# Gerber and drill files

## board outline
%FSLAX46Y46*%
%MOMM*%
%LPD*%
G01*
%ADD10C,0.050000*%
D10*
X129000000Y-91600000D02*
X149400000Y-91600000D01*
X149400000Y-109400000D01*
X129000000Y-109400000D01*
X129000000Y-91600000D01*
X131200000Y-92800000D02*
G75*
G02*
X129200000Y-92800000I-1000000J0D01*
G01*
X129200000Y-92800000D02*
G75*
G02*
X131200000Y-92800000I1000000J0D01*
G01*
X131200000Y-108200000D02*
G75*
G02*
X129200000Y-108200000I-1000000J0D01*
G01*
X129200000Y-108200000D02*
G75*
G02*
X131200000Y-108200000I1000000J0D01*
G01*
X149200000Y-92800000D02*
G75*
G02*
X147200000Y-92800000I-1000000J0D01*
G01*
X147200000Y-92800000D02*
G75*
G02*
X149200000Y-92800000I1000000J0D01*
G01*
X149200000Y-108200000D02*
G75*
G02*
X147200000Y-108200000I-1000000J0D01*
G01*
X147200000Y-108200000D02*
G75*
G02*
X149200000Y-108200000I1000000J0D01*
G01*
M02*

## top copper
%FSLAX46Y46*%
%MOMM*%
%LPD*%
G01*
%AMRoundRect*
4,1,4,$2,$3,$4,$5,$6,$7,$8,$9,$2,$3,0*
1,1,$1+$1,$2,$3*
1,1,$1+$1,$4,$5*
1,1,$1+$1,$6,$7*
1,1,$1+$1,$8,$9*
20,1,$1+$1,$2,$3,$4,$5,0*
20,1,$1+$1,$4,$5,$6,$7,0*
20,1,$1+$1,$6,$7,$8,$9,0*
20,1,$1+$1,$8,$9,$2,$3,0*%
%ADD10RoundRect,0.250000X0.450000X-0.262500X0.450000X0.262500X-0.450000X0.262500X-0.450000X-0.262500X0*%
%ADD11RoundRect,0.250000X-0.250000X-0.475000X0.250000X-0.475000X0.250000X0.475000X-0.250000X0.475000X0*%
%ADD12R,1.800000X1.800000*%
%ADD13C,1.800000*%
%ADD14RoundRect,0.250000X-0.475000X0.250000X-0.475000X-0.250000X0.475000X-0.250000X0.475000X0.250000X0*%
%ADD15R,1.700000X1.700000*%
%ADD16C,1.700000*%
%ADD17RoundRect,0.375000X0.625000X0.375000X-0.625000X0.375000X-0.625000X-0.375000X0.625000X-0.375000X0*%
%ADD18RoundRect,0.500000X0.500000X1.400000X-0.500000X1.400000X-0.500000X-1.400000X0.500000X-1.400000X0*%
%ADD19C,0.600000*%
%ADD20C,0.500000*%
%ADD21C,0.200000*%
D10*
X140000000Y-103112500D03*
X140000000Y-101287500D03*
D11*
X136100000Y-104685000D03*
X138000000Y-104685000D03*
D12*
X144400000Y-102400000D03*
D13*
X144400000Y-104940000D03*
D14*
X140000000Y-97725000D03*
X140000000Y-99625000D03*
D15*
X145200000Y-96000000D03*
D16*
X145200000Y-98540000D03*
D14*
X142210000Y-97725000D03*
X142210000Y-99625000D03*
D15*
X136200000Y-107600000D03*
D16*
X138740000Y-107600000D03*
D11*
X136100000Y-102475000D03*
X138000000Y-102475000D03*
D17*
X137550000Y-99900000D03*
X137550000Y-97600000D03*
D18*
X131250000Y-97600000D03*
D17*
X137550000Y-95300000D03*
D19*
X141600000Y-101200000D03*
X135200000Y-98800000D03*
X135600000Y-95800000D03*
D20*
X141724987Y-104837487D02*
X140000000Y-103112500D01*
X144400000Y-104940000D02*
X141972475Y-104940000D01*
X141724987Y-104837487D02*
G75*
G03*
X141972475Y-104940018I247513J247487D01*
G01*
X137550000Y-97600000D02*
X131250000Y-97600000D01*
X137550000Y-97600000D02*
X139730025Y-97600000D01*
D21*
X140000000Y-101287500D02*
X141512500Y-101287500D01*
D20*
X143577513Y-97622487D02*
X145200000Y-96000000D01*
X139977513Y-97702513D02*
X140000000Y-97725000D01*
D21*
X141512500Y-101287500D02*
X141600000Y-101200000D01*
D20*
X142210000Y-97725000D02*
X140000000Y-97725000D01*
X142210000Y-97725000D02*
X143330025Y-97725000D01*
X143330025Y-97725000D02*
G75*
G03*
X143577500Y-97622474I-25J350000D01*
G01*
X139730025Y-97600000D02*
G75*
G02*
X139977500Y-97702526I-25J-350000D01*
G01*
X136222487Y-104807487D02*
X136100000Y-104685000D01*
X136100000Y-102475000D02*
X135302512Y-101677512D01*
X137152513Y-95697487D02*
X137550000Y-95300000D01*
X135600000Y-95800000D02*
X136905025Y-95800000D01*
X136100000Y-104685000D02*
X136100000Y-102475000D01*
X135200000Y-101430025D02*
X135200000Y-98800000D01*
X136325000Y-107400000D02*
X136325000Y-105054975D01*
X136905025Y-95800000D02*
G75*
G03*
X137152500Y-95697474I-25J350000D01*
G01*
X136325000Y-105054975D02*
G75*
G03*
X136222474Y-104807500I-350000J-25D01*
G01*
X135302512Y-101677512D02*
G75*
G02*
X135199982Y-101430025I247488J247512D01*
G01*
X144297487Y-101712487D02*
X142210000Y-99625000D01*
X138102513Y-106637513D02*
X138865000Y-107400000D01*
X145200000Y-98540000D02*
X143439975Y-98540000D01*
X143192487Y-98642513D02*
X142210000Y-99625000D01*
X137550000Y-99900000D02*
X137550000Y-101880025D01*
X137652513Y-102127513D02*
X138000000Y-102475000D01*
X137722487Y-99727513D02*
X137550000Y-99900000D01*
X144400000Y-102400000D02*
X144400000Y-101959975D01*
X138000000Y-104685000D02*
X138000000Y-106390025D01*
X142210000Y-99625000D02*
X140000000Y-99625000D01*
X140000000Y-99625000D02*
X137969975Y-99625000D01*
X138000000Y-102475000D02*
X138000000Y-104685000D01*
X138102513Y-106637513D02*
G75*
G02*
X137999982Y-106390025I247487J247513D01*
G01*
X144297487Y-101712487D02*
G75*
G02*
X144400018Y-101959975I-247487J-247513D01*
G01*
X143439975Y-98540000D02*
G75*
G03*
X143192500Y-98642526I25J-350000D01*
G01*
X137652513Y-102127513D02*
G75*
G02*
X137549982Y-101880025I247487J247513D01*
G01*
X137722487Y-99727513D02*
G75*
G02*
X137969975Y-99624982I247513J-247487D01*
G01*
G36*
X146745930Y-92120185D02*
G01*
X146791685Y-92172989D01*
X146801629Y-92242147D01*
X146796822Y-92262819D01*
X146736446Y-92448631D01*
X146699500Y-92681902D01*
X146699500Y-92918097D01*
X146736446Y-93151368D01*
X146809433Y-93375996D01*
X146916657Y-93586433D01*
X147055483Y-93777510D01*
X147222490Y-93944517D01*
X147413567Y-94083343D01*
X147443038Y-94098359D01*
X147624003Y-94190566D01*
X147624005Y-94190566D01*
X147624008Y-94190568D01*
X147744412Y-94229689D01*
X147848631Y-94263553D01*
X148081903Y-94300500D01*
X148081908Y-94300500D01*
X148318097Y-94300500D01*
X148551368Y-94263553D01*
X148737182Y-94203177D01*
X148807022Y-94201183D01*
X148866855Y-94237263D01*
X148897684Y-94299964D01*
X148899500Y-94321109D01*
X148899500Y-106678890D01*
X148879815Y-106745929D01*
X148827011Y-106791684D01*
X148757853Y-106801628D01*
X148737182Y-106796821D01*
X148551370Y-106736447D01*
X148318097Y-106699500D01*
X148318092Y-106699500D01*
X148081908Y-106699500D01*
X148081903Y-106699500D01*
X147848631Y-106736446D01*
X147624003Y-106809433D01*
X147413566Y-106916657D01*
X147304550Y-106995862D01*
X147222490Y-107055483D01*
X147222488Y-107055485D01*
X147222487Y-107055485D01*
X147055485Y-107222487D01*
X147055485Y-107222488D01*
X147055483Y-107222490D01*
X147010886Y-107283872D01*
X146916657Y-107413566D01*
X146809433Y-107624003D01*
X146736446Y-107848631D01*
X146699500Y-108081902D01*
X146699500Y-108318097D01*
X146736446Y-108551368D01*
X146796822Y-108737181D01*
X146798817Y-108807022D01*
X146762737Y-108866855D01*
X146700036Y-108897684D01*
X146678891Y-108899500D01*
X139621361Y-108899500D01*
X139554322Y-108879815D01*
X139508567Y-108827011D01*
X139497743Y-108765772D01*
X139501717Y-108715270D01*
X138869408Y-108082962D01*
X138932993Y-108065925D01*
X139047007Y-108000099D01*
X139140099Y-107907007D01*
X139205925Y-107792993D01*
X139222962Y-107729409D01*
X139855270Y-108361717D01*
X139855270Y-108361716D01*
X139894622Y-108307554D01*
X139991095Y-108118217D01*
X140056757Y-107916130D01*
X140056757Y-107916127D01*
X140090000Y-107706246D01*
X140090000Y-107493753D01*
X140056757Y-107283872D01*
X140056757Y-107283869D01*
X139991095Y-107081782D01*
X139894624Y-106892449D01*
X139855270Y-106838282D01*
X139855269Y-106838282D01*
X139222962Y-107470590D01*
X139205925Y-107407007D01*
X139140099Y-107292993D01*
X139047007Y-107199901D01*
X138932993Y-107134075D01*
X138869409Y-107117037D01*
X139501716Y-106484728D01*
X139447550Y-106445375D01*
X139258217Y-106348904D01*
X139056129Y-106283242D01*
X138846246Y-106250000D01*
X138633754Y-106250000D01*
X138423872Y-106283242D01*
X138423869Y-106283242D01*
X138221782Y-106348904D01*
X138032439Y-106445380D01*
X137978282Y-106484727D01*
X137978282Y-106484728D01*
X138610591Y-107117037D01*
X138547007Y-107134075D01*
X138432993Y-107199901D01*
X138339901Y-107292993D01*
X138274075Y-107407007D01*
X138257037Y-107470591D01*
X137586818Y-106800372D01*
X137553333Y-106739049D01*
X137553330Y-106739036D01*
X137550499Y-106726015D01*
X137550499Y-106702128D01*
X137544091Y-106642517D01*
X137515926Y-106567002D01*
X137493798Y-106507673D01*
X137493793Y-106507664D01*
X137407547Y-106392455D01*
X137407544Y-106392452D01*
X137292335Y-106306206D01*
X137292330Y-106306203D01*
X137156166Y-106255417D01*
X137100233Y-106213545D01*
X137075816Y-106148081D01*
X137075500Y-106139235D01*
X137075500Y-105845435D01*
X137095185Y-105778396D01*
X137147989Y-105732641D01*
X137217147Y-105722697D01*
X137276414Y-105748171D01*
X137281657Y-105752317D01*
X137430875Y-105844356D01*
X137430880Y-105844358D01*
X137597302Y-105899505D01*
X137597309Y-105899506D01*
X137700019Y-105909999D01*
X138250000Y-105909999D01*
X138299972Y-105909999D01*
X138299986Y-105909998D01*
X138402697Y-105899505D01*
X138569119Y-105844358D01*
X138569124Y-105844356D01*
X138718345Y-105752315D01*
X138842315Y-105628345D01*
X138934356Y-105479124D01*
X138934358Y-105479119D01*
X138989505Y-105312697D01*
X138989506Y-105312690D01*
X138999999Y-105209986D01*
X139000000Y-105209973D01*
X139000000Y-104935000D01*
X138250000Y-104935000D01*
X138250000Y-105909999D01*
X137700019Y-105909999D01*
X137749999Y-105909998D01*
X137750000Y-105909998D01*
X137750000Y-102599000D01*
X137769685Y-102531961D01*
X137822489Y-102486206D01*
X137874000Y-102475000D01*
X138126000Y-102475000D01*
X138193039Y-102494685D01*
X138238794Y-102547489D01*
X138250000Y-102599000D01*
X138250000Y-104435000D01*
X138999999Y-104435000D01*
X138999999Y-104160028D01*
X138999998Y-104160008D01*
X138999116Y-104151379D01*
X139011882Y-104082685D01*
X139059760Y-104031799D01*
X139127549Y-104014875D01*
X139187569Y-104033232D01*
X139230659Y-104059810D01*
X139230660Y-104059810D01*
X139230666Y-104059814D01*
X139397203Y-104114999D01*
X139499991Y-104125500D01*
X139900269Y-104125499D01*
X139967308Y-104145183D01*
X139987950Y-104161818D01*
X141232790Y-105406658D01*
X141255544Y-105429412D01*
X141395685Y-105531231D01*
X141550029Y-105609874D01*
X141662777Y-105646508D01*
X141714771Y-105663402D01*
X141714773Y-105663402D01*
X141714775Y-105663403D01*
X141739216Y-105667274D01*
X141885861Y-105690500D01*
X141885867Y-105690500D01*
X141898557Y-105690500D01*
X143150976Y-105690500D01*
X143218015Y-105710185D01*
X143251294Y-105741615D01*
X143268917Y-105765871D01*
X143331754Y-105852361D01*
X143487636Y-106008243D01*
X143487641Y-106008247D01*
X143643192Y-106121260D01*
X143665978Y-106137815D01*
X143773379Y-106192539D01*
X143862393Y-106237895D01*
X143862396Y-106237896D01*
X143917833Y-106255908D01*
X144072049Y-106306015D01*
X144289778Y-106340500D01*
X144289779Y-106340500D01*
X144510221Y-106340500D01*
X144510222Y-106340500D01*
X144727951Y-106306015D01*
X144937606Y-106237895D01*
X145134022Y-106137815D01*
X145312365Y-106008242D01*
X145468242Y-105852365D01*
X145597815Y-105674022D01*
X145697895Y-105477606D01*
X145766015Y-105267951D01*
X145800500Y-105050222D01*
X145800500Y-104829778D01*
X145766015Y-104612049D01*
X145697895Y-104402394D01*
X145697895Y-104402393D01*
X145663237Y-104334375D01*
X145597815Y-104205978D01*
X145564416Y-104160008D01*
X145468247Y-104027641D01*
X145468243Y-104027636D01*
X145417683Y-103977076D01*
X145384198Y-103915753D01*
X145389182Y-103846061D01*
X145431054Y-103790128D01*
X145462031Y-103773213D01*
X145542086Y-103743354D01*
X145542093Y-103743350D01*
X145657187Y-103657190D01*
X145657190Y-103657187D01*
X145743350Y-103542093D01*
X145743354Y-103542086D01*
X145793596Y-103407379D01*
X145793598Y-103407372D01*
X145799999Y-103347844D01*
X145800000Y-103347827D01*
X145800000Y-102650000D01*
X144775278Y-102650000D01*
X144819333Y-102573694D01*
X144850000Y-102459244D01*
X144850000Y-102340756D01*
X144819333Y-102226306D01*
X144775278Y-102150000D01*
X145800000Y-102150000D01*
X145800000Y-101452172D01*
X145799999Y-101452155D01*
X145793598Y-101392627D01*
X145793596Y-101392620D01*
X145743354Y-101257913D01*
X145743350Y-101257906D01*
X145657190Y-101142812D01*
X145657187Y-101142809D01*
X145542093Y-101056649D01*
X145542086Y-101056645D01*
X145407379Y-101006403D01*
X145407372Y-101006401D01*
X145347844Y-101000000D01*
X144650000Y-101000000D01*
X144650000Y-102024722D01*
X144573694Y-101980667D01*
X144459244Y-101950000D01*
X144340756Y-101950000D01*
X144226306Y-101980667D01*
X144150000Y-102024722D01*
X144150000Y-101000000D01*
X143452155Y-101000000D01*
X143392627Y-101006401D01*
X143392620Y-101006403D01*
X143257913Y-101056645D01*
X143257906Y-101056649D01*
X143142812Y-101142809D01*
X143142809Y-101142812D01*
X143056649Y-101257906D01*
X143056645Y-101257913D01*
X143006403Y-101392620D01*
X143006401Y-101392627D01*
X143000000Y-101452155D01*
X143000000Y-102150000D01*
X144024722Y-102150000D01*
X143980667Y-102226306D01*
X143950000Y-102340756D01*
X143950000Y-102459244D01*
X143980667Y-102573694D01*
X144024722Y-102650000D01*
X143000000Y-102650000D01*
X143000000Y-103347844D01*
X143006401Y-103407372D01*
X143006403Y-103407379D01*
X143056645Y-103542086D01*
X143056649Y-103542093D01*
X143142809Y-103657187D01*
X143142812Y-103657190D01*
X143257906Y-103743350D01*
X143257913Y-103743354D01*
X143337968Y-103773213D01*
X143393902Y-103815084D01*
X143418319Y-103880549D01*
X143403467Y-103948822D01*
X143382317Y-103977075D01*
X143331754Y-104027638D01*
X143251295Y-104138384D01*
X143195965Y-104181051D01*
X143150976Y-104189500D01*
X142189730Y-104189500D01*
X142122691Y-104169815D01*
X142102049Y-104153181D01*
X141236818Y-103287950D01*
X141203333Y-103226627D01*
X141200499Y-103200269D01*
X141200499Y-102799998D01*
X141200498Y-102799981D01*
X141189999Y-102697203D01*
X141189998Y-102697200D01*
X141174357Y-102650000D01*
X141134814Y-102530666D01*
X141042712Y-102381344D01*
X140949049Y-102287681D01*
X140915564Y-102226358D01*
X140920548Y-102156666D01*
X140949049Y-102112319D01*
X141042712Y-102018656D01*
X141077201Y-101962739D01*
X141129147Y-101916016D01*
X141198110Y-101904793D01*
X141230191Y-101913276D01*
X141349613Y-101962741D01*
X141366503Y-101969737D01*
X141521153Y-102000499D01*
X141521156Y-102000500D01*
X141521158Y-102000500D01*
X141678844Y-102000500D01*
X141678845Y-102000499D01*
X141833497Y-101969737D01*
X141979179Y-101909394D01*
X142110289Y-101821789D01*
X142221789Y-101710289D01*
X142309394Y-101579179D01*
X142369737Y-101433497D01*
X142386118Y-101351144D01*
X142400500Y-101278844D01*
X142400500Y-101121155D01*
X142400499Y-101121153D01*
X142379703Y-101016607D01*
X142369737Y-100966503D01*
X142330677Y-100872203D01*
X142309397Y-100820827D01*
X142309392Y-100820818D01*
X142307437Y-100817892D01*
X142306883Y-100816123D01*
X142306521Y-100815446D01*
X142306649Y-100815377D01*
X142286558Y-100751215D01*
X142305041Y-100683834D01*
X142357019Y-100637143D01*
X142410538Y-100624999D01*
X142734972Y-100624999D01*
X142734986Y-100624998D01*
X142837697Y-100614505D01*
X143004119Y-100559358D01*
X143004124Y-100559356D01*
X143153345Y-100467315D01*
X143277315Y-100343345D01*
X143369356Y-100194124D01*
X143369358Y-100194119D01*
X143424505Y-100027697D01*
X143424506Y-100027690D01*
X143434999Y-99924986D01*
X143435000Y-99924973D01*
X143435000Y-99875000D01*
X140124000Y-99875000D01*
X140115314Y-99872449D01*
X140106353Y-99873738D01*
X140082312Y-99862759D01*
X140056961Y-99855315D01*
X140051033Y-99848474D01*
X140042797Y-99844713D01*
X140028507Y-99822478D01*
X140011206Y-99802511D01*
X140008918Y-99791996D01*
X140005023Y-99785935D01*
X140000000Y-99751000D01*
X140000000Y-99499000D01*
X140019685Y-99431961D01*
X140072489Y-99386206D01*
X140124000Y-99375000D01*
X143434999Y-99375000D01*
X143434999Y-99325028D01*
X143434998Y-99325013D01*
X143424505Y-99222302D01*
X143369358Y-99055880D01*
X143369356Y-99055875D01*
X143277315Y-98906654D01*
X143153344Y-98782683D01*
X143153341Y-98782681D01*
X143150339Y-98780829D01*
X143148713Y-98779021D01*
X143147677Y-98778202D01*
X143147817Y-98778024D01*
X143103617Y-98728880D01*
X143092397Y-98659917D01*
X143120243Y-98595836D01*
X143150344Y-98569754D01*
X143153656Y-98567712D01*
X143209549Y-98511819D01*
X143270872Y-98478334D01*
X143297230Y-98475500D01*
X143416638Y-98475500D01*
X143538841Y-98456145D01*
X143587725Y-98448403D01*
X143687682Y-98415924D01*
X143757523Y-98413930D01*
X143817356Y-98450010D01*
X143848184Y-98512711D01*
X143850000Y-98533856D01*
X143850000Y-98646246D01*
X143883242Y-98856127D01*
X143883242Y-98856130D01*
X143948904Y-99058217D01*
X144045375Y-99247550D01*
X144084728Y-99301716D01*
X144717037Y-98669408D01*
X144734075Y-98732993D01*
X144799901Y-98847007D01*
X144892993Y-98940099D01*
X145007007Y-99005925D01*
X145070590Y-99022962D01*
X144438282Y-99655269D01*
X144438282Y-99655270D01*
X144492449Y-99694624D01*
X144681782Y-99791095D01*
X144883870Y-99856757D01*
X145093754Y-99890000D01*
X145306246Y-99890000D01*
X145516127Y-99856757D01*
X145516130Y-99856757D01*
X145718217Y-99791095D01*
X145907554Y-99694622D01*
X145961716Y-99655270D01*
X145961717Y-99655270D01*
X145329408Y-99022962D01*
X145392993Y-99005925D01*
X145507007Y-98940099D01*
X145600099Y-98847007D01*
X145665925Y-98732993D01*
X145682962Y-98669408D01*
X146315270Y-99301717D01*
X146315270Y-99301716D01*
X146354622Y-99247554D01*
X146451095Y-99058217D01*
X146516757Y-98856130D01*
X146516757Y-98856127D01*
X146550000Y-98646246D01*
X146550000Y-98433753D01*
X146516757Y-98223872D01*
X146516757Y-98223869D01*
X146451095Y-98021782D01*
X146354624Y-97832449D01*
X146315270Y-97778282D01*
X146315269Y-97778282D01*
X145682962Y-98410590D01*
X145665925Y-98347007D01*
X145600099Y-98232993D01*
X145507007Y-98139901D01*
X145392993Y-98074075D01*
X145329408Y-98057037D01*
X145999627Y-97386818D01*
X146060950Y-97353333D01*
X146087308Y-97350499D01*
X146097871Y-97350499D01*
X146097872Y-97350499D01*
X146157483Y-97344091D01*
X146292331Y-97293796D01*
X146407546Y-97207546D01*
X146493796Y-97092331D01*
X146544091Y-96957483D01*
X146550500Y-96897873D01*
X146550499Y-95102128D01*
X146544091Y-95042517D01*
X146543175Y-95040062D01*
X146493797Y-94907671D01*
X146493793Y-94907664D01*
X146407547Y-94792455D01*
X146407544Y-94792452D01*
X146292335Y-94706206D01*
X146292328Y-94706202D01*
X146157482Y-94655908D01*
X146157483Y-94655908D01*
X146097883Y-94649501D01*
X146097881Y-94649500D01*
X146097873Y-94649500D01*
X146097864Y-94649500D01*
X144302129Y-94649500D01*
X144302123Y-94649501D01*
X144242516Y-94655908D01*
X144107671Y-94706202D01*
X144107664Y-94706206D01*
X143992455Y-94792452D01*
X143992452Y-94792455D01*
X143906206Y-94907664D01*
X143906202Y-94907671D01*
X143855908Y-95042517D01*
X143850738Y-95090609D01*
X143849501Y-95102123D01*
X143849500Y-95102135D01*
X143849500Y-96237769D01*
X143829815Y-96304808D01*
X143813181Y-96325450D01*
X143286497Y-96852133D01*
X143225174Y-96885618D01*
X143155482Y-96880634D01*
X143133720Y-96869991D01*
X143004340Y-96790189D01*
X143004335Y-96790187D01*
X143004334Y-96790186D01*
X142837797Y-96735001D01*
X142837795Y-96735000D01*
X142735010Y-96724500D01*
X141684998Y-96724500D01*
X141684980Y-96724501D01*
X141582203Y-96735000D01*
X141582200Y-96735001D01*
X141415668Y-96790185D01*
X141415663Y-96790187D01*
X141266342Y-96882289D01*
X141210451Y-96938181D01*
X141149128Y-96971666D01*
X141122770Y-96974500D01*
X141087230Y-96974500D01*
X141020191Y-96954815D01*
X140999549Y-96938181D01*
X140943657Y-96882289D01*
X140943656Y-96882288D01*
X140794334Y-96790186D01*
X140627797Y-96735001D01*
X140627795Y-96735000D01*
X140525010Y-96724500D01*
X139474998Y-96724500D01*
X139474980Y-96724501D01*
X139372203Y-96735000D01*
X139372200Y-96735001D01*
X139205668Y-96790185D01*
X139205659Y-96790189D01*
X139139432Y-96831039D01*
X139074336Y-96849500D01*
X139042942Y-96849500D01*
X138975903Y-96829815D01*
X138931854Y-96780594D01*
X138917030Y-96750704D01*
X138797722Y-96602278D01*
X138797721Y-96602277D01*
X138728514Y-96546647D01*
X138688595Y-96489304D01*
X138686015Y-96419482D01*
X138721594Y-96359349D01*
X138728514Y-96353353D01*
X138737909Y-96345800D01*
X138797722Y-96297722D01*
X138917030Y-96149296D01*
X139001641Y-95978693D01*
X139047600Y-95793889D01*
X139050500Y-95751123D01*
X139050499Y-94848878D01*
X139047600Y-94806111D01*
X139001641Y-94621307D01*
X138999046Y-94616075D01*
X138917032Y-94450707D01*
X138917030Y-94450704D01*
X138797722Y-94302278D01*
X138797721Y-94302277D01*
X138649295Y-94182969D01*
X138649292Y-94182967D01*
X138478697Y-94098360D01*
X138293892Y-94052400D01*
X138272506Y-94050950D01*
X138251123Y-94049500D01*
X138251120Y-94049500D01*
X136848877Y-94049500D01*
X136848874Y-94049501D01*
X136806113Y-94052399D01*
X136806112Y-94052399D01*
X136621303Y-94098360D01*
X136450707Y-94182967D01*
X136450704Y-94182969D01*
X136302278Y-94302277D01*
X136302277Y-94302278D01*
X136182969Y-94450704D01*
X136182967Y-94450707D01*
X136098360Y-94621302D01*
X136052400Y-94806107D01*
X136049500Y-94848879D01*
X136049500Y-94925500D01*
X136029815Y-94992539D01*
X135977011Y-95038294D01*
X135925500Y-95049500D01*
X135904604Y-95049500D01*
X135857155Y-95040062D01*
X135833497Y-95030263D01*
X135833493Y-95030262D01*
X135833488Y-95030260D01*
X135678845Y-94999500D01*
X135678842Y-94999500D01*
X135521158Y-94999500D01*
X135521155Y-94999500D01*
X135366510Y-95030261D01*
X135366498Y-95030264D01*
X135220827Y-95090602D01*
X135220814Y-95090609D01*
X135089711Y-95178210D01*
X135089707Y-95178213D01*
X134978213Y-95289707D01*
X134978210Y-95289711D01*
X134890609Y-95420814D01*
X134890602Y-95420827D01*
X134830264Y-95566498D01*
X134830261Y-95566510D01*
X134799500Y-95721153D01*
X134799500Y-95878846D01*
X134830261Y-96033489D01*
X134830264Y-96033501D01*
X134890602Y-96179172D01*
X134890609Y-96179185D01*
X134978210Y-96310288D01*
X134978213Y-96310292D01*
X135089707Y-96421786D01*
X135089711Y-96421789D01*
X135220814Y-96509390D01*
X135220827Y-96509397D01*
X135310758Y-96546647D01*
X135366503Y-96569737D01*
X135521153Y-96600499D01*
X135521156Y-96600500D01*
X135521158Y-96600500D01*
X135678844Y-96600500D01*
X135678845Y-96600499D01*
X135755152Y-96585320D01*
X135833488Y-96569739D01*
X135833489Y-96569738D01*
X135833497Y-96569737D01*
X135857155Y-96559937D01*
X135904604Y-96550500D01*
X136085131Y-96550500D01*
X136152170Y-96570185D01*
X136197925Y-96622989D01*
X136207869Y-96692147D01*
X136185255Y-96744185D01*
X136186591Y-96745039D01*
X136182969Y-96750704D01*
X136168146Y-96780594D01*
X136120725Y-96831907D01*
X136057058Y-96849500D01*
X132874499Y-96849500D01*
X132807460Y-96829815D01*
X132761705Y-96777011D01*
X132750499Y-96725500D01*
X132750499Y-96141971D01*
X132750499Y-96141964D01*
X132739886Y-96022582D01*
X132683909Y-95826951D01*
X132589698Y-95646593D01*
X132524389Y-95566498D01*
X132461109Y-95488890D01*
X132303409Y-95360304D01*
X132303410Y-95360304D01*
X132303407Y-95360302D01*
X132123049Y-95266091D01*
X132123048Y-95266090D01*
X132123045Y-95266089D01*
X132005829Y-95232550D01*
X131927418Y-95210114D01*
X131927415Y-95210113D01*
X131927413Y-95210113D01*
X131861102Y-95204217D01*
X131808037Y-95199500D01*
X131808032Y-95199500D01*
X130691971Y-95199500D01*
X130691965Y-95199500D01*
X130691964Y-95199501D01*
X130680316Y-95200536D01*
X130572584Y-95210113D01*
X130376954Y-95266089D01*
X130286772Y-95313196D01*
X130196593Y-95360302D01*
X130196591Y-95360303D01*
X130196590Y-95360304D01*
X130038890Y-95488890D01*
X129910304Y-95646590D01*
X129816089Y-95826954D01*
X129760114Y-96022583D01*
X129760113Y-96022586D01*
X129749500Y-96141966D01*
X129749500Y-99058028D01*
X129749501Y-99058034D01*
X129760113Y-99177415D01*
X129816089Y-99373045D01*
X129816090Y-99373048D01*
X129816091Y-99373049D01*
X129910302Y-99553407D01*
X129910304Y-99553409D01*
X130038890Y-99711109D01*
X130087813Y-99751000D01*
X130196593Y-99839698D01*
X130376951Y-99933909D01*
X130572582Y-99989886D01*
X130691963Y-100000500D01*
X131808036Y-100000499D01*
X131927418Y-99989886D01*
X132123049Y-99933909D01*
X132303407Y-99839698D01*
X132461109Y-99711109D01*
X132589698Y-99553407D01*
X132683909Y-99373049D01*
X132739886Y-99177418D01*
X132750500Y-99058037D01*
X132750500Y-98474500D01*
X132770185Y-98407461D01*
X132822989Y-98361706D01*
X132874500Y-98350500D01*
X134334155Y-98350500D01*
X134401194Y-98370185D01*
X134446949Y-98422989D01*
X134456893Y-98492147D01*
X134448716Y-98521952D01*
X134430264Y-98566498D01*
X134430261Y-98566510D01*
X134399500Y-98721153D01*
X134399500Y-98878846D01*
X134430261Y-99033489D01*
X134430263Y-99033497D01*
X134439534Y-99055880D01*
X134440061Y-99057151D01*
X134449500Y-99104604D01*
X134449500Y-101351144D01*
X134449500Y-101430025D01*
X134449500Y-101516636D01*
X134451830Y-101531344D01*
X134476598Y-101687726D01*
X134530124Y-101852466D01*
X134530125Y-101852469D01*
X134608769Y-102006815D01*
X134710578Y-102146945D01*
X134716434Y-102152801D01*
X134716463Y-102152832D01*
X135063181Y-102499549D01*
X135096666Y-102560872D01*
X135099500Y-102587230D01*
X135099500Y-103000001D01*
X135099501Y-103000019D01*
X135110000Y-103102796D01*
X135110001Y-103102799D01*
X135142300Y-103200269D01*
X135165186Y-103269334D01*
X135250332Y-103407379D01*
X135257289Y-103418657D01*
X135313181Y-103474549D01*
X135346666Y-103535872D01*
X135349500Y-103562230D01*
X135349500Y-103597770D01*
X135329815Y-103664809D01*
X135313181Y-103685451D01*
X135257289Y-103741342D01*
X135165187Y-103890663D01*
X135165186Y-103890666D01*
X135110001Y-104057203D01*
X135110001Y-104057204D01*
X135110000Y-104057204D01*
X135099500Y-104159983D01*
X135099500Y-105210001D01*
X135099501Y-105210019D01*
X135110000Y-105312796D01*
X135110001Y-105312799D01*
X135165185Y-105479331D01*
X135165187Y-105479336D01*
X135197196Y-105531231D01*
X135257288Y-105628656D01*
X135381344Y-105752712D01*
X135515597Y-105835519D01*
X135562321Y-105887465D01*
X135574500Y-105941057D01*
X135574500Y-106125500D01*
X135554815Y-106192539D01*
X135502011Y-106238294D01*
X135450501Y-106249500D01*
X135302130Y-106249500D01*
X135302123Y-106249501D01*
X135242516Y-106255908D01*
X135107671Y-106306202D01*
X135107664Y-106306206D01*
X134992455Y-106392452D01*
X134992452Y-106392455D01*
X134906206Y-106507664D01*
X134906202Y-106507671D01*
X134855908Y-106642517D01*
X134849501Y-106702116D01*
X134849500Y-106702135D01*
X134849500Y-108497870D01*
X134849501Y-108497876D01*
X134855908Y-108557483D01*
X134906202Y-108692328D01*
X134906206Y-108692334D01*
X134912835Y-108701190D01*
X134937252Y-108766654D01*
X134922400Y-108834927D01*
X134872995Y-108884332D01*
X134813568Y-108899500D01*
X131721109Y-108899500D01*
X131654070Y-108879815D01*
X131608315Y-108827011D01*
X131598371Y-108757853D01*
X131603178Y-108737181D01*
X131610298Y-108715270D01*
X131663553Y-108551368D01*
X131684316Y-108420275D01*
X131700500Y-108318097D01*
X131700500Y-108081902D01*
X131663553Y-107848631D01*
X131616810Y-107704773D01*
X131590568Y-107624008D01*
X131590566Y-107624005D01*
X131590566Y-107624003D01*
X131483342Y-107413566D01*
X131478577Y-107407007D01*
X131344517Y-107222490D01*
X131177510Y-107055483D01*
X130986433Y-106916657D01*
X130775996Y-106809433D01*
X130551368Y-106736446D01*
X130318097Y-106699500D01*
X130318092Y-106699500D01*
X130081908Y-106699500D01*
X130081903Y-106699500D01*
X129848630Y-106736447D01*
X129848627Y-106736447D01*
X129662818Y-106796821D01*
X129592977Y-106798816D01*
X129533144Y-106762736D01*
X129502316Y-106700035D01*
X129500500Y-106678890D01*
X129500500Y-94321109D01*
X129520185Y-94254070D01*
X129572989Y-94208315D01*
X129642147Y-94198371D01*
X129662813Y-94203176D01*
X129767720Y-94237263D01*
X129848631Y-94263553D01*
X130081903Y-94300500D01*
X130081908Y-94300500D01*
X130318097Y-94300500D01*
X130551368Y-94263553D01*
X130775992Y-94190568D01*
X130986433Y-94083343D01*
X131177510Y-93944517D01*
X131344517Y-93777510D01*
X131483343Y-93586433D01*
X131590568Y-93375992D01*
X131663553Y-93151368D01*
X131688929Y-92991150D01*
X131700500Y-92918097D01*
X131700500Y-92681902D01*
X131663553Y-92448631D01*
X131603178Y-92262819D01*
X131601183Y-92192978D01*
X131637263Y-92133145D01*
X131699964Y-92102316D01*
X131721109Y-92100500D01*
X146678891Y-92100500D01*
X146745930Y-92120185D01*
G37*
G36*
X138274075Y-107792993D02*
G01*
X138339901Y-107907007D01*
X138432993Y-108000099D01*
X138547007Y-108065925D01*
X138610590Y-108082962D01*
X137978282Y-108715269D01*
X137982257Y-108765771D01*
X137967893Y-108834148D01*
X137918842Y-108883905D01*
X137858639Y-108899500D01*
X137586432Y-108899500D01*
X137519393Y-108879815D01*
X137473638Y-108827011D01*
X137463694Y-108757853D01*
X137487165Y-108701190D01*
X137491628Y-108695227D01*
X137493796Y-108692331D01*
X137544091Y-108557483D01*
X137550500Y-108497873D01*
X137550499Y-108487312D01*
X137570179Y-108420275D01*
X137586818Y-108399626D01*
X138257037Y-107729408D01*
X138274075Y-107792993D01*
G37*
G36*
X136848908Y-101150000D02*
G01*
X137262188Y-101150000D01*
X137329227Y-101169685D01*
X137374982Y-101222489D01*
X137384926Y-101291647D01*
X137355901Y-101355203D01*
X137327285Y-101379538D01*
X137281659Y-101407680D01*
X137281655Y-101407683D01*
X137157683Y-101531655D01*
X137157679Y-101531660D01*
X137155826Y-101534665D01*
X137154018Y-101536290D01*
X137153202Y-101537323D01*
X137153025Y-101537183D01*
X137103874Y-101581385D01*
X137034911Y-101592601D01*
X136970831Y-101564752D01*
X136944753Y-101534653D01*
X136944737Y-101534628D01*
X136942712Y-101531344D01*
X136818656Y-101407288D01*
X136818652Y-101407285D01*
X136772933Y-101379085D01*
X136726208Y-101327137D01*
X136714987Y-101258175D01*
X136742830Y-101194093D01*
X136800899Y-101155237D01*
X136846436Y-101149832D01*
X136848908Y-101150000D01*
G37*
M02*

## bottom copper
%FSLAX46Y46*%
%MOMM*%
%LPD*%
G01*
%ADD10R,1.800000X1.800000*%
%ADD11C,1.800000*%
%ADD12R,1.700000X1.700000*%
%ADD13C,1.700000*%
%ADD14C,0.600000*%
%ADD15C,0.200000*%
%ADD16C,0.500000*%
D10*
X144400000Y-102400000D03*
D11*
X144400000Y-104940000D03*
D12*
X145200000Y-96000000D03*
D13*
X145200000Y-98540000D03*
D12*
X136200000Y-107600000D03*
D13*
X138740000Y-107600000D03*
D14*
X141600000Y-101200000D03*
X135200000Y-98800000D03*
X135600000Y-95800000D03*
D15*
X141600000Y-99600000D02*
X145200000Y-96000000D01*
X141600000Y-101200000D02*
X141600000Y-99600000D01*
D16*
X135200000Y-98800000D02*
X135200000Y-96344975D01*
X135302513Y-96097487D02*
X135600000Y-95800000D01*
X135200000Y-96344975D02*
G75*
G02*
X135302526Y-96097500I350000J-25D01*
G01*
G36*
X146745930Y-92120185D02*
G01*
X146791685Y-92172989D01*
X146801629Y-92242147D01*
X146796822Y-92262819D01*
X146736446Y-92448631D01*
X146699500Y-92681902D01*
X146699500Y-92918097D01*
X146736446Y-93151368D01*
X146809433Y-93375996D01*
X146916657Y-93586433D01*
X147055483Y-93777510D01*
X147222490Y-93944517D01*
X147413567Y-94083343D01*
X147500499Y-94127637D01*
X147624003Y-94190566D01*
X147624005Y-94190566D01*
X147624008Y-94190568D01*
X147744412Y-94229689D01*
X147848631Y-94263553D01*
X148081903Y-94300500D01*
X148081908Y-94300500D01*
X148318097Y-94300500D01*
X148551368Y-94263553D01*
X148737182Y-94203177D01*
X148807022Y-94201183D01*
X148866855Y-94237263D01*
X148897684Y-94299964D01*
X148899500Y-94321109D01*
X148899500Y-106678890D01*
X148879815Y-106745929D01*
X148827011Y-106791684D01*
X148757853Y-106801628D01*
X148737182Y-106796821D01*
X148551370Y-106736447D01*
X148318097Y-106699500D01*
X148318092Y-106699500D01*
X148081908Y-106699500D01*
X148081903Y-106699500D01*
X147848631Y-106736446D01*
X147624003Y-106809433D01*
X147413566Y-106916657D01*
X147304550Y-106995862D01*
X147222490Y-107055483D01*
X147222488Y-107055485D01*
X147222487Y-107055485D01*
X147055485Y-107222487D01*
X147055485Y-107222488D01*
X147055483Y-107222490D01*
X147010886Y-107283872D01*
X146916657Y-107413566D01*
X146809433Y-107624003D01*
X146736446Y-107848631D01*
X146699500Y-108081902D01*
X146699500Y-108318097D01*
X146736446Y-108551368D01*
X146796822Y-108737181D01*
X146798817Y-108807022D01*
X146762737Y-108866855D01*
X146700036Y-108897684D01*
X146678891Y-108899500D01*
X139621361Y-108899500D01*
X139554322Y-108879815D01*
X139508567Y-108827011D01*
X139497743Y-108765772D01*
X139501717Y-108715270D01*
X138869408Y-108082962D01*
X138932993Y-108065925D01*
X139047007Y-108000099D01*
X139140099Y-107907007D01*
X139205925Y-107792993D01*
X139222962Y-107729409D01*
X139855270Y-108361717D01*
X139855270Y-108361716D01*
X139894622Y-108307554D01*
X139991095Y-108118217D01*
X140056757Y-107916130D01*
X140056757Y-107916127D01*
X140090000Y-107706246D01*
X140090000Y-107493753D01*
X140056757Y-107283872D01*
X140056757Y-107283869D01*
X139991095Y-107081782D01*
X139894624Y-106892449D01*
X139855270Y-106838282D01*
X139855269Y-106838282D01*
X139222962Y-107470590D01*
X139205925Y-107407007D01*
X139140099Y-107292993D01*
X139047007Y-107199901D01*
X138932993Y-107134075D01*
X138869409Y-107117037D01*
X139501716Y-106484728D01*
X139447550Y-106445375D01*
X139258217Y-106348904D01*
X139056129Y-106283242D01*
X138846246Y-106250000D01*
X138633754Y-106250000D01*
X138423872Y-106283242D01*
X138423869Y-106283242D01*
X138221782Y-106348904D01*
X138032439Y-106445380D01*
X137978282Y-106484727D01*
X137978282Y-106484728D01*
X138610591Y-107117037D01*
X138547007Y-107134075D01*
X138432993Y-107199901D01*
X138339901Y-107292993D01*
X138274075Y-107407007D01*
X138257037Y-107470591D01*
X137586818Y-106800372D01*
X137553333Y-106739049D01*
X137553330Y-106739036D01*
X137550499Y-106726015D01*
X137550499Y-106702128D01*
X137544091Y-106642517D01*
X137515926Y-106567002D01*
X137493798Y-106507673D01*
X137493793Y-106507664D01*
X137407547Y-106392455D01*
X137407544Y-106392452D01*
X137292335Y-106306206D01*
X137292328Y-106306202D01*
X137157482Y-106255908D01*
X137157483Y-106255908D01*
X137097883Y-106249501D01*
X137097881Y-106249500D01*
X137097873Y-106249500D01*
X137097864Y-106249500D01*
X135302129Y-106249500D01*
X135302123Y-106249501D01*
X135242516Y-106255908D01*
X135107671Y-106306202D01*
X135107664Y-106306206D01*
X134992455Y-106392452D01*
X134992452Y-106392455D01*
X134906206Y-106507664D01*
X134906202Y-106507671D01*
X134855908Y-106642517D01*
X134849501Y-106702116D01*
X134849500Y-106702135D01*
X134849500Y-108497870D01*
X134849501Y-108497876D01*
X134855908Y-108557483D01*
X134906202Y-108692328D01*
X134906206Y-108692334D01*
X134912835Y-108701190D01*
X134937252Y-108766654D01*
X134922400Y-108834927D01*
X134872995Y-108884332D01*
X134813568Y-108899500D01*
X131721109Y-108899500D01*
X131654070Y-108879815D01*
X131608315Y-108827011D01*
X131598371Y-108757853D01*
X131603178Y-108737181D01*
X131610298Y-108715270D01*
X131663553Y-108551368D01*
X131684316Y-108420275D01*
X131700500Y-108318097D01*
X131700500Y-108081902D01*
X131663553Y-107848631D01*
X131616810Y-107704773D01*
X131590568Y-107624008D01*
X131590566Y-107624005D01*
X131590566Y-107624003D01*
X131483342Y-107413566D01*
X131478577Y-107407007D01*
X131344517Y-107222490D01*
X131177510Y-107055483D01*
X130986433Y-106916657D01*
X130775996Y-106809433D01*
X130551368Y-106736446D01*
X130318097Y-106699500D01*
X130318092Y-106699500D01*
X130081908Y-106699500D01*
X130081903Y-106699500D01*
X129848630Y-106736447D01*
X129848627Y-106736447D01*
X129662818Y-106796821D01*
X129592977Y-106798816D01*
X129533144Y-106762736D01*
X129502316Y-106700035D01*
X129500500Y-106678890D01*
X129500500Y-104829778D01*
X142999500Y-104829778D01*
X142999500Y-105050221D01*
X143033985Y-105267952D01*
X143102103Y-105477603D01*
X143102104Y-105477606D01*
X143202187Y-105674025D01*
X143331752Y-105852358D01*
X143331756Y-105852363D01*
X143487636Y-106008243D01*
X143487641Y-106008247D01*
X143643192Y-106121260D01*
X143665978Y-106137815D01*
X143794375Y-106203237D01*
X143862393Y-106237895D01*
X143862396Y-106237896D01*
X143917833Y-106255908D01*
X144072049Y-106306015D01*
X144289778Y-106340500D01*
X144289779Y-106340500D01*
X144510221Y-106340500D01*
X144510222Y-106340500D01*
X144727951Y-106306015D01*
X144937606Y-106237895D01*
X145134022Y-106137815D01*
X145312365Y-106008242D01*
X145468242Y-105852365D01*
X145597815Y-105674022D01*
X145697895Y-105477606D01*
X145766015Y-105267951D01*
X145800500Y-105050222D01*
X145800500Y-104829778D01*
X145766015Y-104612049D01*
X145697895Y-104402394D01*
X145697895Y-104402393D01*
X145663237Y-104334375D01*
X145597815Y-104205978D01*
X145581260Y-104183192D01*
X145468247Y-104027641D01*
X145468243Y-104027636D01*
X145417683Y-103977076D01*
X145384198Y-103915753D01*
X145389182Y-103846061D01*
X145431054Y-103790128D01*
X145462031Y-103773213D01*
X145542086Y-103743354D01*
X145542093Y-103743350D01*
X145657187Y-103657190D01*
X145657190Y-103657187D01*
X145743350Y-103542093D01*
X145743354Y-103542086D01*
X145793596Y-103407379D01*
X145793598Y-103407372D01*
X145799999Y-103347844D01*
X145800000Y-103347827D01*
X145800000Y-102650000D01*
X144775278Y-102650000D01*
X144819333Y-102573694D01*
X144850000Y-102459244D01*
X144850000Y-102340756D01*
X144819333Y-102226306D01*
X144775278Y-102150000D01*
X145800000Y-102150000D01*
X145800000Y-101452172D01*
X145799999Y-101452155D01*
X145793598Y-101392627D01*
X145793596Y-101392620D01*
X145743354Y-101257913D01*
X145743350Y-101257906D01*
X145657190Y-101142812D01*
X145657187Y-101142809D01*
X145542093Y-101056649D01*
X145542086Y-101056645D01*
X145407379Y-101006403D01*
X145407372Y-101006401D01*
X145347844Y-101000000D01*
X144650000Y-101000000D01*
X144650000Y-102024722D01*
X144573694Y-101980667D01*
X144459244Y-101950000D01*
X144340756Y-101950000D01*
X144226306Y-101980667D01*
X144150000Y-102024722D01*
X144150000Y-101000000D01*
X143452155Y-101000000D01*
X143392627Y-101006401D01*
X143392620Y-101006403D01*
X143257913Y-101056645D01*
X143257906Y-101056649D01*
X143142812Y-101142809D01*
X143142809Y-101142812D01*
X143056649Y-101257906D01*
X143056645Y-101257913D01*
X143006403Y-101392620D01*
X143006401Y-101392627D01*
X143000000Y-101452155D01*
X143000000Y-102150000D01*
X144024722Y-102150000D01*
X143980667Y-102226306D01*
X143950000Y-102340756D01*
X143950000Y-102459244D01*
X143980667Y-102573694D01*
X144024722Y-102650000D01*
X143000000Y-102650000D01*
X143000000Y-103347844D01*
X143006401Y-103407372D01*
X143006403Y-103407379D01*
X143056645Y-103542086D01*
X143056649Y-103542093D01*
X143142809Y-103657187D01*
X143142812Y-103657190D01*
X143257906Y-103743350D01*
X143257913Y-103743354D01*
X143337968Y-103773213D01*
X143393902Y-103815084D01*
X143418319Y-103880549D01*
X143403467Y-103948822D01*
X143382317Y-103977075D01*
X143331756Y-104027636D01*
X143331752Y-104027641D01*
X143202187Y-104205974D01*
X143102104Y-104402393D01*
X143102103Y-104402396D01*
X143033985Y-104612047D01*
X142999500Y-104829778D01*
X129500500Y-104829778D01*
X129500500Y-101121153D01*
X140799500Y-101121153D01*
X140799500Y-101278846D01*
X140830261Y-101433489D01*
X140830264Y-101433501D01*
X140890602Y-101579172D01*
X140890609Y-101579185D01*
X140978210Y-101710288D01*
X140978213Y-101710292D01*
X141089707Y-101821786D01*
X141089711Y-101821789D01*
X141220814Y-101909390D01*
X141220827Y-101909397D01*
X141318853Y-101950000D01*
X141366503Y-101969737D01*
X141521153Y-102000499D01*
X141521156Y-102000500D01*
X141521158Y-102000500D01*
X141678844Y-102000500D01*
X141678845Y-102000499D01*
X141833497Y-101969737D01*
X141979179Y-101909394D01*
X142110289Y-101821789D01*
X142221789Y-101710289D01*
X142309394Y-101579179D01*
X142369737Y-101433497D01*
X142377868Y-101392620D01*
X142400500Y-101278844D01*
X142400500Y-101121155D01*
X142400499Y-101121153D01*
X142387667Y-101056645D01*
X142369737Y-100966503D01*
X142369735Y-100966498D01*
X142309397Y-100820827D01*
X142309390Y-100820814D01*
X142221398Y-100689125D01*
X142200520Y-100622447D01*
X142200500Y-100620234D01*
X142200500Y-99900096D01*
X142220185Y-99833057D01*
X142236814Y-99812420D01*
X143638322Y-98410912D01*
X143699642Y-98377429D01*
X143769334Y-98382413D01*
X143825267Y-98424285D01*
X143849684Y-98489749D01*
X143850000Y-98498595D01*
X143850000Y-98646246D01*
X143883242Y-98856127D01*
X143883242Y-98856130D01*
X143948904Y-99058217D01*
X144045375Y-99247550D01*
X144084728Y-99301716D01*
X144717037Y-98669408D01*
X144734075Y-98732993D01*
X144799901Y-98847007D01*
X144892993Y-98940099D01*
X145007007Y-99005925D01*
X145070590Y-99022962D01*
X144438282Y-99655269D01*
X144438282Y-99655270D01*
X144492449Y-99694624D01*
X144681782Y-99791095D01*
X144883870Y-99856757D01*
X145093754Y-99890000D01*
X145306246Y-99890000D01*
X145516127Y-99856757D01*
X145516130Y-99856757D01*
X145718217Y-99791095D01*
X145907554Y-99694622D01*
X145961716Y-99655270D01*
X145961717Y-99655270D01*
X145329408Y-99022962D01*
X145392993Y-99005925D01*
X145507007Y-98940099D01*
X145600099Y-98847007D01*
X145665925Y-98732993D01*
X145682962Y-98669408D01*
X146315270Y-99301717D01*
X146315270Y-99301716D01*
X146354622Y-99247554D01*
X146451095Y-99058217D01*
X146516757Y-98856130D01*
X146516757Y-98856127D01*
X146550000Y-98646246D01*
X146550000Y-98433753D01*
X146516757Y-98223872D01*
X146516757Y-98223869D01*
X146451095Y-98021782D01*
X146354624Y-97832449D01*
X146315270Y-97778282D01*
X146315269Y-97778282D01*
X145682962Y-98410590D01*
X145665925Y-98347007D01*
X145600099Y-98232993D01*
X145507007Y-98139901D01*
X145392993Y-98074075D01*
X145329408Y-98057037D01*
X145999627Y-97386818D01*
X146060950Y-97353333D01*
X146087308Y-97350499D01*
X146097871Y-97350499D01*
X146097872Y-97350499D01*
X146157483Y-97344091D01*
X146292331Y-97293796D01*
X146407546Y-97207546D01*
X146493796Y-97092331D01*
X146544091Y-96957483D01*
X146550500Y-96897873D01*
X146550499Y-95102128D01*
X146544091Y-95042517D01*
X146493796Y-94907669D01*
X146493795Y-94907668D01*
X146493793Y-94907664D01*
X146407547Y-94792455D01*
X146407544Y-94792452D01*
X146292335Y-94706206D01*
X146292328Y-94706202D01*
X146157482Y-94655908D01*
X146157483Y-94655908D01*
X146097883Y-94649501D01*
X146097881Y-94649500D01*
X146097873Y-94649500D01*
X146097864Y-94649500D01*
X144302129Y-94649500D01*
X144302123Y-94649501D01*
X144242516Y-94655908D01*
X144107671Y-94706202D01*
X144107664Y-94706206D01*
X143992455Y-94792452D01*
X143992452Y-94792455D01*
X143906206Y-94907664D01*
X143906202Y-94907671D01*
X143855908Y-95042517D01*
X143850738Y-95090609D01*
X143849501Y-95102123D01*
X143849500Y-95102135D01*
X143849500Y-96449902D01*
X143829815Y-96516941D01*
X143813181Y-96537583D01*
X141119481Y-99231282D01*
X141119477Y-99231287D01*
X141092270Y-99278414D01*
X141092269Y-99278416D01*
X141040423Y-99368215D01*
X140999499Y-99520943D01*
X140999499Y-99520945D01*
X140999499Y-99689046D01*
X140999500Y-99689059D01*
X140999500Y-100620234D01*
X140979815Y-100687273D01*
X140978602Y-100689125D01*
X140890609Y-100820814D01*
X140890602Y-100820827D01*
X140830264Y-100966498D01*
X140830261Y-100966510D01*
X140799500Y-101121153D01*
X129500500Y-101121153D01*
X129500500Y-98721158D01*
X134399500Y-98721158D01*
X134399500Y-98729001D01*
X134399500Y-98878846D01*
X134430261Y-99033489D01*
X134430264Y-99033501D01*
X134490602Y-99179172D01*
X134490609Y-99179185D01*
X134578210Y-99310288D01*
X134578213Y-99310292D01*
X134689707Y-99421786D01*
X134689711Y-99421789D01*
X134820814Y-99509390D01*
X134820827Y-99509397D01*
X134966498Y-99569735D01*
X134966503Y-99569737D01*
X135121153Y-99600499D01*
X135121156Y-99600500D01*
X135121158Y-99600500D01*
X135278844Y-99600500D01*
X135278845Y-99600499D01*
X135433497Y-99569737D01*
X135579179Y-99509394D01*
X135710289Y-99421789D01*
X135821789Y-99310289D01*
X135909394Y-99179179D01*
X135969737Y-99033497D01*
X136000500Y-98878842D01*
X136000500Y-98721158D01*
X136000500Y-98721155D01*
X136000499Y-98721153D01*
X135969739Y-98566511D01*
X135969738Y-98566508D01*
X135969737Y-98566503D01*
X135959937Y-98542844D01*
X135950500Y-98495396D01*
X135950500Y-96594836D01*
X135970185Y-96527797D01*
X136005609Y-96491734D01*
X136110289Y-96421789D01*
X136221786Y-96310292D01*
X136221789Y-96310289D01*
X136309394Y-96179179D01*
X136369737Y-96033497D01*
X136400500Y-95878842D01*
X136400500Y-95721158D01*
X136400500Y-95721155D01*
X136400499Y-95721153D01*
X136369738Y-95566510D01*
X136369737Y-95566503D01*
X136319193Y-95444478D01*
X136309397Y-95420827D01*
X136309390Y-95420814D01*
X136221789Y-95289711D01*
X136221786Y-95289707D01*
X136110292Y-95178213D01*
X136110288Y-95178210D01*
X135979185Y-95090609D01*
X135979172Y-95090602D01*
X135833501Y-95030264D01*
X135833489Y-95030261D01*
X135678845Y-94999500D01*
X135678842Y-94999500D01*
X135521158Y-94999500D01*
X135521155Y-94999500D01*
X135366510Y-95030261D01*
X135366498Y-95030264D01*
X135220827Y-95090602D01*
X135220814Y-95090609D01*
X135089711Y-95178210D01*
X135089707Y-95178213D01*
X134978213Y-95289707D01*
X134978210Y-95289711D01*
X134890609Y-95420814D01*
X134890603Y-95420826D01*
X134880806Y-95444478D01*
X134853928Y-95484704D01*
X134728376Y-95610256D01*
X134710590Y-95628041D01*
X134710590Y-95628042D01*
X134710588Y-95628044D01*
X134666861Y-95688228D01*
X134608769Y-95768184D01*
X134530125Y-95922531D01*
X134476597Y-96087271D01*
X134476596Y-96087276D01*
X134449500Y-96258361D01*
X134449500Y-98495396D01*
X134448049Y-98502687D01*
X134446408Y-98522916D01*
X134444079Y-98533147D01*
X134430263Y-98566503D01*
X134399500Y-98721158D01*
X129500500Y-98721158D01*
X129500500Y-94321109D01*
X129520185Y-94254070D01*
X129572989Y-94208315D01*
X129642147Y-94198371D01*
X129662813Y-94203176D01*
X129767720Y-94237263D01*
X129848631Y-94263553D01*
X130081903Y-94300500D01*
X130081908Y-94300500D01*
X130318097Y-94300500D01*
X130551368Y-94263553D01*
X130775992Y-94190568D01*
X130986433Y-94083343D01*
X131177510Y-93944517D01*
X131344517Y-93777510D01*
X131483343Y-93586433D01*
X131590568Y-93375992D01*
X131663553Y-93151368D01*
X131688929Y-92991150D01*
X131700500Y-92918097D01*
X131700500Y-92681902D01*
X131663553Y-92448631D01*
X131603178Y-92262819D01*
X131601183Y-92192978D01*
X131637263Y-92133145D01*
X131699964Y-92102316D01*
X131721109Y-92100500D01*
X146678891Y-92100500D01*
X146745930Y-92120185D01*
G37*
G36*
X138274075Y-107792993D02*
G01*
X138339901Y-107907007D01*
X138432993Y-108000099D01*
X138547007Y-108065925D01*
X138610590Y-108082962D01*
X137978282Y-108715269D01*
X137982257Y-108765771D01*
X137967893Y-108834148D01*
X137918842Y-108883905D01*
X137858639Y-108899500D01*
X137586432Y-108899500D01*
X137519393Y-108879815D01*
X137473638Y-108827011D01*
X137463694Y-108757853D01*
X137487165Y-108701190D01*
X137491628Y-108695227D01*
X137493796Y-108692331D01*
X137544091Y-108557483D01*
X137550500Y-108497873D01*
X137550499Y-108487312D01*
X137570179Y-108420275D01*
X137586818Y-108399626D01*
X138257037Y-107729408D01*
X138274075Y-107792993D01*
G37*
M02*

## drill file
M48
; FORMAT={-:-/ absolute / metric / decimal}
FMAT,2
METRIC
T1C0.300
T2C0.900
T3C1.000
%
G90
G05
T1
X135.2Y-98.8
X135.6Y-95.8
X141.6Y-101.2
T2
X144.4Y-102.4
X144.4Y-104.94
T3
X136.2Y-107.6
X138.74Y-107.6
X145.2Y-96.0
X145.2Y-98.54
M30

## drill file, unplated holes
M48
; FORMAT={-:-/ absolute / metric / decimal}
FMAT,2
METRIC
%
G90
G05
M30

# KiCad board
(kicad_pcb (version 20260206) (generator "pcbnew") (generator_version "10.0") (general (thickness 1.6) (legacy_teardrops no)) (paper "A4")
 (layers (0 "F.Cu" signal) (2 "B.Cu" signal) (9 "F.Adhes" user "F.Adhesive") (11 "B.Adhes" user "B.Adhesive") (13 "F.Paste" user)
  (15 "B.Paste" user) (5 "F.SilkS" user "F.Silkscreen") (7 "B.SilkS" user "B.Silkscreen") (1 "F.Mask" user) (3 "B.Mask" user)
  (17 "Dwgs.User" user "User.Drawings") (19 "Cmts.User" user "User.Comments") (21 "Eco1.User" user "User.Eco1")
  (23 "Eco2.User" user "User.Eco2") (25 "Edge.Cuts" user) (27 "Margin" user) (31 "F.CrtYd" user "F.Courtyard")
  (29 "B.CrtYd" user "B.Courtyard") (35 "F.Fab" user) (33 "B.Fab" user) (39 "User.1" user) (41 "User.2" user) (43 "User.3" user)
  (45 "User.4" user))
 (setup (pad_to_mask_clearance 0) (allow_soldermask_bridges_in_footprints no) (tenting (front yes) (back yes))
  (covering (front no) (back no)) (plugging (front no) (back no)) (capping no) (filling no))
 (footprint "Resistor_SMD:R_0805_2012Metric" (layer "F.Cu") (at 140 102.2 90)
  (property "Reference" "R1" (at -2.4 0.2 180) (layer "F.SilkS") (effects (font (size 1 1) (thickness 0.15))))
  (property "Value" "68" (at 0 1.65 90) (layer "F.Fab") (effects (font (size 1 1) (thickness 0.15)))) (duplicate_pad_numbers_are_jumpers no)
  (pad "1" smd roundrect (at -0.9125 0 90) (size 1.025 1.4) (layers "F.Cu" "F.Mask" "F.Paste") (roundrect_rratio 0.243902)
   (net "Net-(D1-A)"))
  (pad "2" smd roundrect (at 0.9125 0 90) (size 1.025 1.4) (layers "F.Cu" "F.Mask" "F.Paste") (roundrect_rratio 0.243902) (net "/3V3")))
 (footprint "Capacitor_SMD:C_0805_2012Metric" (layer "F.Cu") (at 137.05 104.685)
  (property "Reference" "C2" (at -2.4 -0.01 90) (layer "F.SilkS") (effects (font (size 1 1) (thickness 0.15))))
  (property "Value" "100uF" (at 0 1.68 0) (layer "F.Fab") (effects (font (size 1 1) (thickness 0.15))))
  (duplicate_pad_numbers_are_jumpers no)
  (pad "1" smd roundrect (at -0.95 0) (size 1 1.45) (layers "F.Cu" "F.Mask" "F.Paste") (roundrect_rratio 0.25) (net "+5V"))
  (pad "2" smd roundrect (at 0.95 0) (size 1 1.45) (layers "F.Cu" "F.Mask" "F.Paste") (roundrect_rratio 0.25) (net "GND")))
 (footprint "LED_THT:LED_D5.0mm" (layer "F.Cu") (at 144.4 102.4 -90)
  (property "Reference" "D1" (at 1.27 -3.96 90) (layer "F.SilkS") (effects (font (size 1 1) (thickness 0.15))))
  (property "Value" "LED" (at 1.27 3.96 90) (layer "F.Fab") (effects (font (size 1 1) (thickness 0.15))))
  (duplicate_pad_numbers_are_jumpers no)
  (pad "1" thru_hole rect (at 0 0 270) (size 1.8 1.8) (drill 0.9) (layers "*.Cu" "*.Mask") (remove_unused_layers no) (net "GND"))
  (pad "2" thru_hole circle (at 2.54 0 270) (size 1.8 1.8) (drill 0.9) (layers "*.Cu" "*.Mask") (remove_unused_layers no) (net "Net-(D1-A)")))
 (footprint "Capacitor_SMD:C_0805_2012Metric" (layer "F.Cu") (at 140 98.675 -90)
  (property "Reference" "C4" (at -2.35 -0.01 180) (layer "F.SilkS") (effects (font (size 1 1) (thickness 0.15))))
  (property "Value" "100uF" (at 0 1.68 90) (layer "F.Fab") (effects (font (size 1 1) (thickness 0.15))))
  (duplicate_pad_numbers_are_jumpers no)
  (pad "1" smd roundrect (at -0.95 0 270) (size 1 1.45) (layers "F.Cu" "F.Mask" "F.Paste") (roundrect_rratio 0.25) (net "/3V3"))
  (pad "2" smd roundrect (at 0.95 0 270) (size 1 1.45) (layers "F.Cu" "F.Mask" "F.Paste") (roundrect_rratio 0.25) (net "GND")))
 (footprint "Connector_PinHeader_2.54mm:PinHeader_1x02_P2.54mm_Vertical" (layer "F.Cu") (at 145.2 96)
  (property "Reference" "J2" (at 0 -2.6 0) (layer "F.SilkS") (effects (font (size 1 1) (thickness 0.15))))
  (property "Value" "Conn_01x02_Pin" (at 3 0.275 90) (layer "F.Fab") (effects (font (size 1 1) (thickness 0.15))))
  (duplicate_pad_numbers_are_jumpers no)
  (pad "1" thru_hole rect (at 0 0) (size 1.7 1.7) (drill 1) (layers "*.Cu" "*.Mask") (remove_unused_layers no) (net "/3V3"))
  (pad "2" thru_hole circle (at 0 2.54) (size 1.7 1.7) (drill 1) (layers "*.Cu" "*.Mask") (remove_unused_layers no) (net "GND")))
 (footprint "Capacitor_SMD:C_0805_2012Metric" (layer "F.Cu") (at 142.21 98.675 -90)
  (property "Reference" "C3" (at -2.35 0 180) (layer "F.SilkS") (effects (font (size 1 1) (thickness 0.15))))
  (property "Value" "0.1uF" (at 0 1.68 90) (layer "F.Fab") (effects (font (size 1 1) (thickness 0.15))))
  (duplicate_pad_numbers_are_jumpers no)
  (pad "1" smd roundrect (at -0.95 0 270) (size 1 1.45) (layers "F.Cu" "F.Mask" "F.Paste") (roundrect_rratio 0.25) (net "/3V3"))
  (pad "2" smd roundrect (at 0.95 0 270) (size 1 1.45) (layers "F.Cu" "F.Mask" "F.Paste") (roundrect_rratio 0.25) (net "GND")))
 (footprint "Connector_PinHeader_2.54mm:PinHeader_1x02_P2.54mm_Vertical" (layer "F.Cu") (at 136.2 107.6 90)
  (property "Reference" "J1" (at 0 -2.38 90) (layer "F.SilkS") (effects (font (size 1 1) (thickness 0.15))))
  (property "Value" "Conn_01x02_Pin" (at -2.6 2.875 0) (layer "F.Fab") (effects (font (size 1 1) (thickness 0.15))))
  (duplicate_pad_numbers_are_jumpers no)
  (pad "1" thru_hole rect (at 0 0 90) (size 1.7 1.7) (drill 1) (layers "*.Cu" "*.Mask") (remove_unused_layers no) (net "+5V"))
  (pad "2" thru_hole circle (at 0 2.54 90) (size 1.7 1.7) (drill 1) (layers "*.Cu" "*.Mask") (remove_unused_layers no) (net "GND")))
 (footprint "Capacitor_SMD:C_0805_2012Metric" (layer "F.Cu") (at 137.05 102.475)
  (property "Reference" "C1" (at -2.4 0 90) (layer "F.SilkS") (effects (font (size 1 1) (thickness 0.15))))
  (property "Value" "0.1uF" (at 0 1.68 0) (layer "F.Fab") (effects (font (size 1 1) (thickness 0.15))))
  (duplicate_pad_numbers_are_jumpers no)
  (pad "1" smd roundrect (at -0.95 0) (size 1 1.45) (layers "F.Cu" "F.Mask" "F.Paste") (roundrect_rratio 0.25) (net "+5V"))
  (pad "2" smd roundrect (at 0.95 0) (size 1 1.45) (layers "F.Cu" "F.Mask" "F.Paste") (roundrect_rratio 0.25) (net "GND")))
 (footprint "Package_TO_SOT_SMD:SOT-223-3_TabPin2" (layer "F.Cu") (at 134.4 97.6 180)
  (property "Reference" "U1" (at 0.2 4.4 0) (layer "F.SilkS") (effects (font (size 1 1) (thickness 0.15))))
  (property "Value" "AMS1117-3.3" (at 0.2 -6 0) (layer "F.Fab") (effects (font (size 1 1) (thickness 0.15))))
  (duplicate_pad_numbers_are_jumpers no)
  (pad "1" smd roundrect (at -3.15 -2.3 180) (size 2 1.5) (layers "F.Cu" "F.Mask" "F.Paste") (roundrect_rratio 0.25) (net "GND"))
  (pad "2" smd roundrect (at -3.15 0 180) (size 2 1.5) (layers "F.Cu" "F.Mask" "F.Paste") (roundrect_rratio 0.25) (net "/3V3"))
  (pad "2" smd roundrect (at 3.15 0 180) (size 2 3.8) (layers "F.Cu" "F.Mask" "F.Paste") (roundrect_rratio 0.25) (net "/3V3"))
  (pad "3" smd roundrect (at -3.15 2.3 180) (size 2 1.5) (layers "F.Cu" "F.Mask" "F.Paste") (roundrect_rratio 0.25) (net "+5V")))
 (gr_rect (start 129 91.6) (end 149.4 109.4) (stroke (width 0.05) (type default)) (fill no) (layer "Edge.Cuts"))
 (gr_circle (center 130.2 92.8) (end 131.2 92.8) (stroke (width 0.05) (type default)) (fill no) (layer "Edge.Cuts"))
 (gr_circle (center 130.2 108.2) (end 131.2 108.2) (stroke (width 0.05) (type default)) (fill no) (layer "Edge.Cuts"))
 (gr_circle (center 148.2 92.8) (end 149.2 92.8) (stroke (width 0.05) (type default)) (fill no) (layer "Edge.Cuts"))
 (gr_circle (center 148.2 108.2) (end 149.2 108.2) (stroke (width 0.05) (type default)) (fill no) (layer "Edge.Cuts"))
 (segment (start 141.724987 104.837487) (end 140 103.1125) (width 0.5) (layer "F.Cu") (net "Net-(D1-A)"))
 (segment (start 144.4 104.94) (end 141.972475 104.94) (width 0.5) (layer "F.Cu") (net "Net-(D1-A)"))
 (arc (start 141.724987 104.837487) (mid 141.838535 104.913358) (end 141.972475 104.94) (width 0.5) (layer "F.Cu") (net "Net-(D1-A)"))
 (segment (start 137.55 97.6) (end 131.25 97.6) (width 0.5) (layer "F.Cu") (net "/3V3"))
 (segment (start 137.55 97.6) (end 139.730025 97.6) (width 0.5) (layer "F.Cu") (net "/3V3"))
 (segment (start 140 101.2875) (end 141.5125 101.2875) (width 0.2) (layer "F.Cu") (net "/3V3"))
 (segment (start 143.577513 97.622487) (end 145.2 96) (width 0.5) (layer "F.Cu") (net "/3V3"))
 (segment (start 139.977513 97.702513) (end 140 97.725) (width 0.5) (layer "F.Cu") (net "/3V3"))
 (segment (start 141.5125 101.2875) (end 141.6 101.2) (width 0.2) (layer "F.Cu") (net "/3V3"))
 (segment (start 142.21 97.725) (end 140 97.725) (width 0.5) (layer "F.Cu") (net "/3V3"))
 (segment (start 142.21 97.725) (end 143.330025 97.725) (width 0.5) (layer "F.Cu") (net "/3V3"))
 (via (at 141.6 101.2) (size 0.6) (drill 0.3) (layers "F.Cu" "B.Cu") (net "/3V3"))
 (arc (start 143.330025 97.725) (mid 143.463965 97.698358) (end 143.577513 97.622487) (width 0.5) (layer "F.Cu") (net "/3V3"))
 (arc (start 139.730025 97.6) (mid 139.863965 97.626642) (end 139.977513 97.702513) (width 0.5) (layer "F.Cu") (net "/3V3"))
 (segment (start 141.6 99.6) (end 145.2 96) (width 0.2) (layer "B.Cu") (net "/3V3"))
 (segment (start 141.6 101.2) (end 141.6 99.6) (width 0.2) (layer "B.Cu") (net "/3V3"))
 (segment (start 136.222487 104.807487) (end 136.1 104.685) (width 0.5) (layer "F.Cu") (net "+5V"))
 (segment (start 136.1 102.475) (end 135.302512 101.677512) (width 0.5) (layer "F.Cu") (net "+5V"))
 (segment (start 137.152513 95.697487) (end 137.55 95.3) (width 0.5) (layer "F.Cu") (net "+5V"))
 (segment (start 135.6 95.8) (end 136.905025 95.8) (width 0.5) (layer "F.Cu") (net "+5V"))
 (segment (start 136.1 104.685) (end 136.1 102.475) (width 0.5) (layer "F.Cu") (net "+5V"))
 (segment (start 135.2 101.430025) (end 135.2 98.8) (width 0.5) (layer "F.Cu") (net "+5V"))
 (segment (start 136.325 107.4) (end 136.325 105.054975) (width 0.5) (layer "F.Cu") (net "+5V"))
 (via (at 135.2 98.8) (size 0.6) (drill 0.3) (layers "F.Cu" "B.Cu") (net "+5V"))
 (via (at 135.6 95.8) (size 0.6) (drill 0.3) (layers "F.Cu" "B.Cu") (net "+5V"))
 (arc (start 136.905025 95.8) (mid 137.038965 95.773358) (end 137.152513 95.697487) (width 0.5) (layer "F.Cu") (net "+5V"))
 (arc (start 136.325 105.054975) (mid 136.298358 104.921035) (end 136.222487 104.807487) (width 0.5) (layer "F.Cu") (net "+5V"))
 (arc (start 135.302512 101.677512) (mid 135.226642 101.563964) (end 135.2 101.430025) (width 0.5) (layer "F.Cu") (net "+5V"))
 (segment (start 135.2 98.8) (end 135.2 96.344975) (width 0.5) (layer "B.Cu") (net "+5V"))
 (segment (start 135.302513 96.097487) (end 135.6 95.8) (width 0.5) (layer "B.Cu") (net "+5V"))
 (arc (start 135.2 96.344975) (mid 135.226642 96.211035) (end 135.302513 96.097487) (width 0.5) (layer "B.Cu") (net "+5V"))
 (segment (start 144.297487 101.712487) (end 142.21 99.625) (width 0.5) (layer "F.Cu") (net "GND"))
 (segment (start 138.102513 106.637513) (end 138.865 107.4) (width 0.5) (layer "F.Cu") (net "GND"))
 (segment (start 145.2 98.54) (end 143.439975 98.54) (width 0.5) (layer "F.Cu") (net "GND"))
 (segment (start 143.192487 98.642513) (end 142.21 99.625) (width 0.5) (layer "F.Cu") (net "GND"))
 (segment (start 137.55 99.9) (end 137.55 101.880025) (width 0.5) (layer "F.Cu") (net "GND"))
 (segment (start 137.652513 102.127513) (end 138 102.475) (width 0.5) (layer "F.Cu") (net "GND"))
 (segment (start 137.722487 99.727513) (end 137.55 99.9) (width 0.5) (layer "F.Cu") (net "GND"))
 (segment (start 144.4 102.4) (end 144.4 101.959975) (width 0.5) (layer "F.Cu") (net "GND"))
 (segment (start 138 104.685) (end 138 106.390025) (width 0.5) (layer "F.Cu") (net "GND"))
 (segment (start 142.21 99.625) (end 140 99.625) (width 0.5) (layer "F.Cu") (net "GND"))
 (segment (start 140 99.625) (end 137.969975 99.625) (width 0.5) (layer "F.Cu") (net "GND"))
 (segment (start 138 102.475) (end 138 104.685) (width 0.5) (layer "F.Cu") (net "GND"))
 (arc (start 138.102513 106.637513) (mid 138.026642 106.523965) (end 138 106.390025) (width 0.5) (layer "F.Cu") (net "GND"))
 (arc (start 144.297487 101.712487) (mid 144.373358 101.826035) (end 144.4 101.959975) (width 0.5) (layer "F.Cu") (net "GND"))
 (arc (start 143.439975 98.54) (mid 143.306035 98.566642) (end 143.192487 98.642513) (width 0.5) (layer "F.Cu") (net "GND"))
 (arc (start 137.652513 102.127513) (mid 137.576642 102.013965) (end 137.55 101.880025) (width 0.5) (layer "F.Cu") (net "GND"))
 (arc (start 137.722487 99.727513) (mid 137.836035 99.651642) (end 137.969975 99.625) (width 0.5) (layer "F.Cu") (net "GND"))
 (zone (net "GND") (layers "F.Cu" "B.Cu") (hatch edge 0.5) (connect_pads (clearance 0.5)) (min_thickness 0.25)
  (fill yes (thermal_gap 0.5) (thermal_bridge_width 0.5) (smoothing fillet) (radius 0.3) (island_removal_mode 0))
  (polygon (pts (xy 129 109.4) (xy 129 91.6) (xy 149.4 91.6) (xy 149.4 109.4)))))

